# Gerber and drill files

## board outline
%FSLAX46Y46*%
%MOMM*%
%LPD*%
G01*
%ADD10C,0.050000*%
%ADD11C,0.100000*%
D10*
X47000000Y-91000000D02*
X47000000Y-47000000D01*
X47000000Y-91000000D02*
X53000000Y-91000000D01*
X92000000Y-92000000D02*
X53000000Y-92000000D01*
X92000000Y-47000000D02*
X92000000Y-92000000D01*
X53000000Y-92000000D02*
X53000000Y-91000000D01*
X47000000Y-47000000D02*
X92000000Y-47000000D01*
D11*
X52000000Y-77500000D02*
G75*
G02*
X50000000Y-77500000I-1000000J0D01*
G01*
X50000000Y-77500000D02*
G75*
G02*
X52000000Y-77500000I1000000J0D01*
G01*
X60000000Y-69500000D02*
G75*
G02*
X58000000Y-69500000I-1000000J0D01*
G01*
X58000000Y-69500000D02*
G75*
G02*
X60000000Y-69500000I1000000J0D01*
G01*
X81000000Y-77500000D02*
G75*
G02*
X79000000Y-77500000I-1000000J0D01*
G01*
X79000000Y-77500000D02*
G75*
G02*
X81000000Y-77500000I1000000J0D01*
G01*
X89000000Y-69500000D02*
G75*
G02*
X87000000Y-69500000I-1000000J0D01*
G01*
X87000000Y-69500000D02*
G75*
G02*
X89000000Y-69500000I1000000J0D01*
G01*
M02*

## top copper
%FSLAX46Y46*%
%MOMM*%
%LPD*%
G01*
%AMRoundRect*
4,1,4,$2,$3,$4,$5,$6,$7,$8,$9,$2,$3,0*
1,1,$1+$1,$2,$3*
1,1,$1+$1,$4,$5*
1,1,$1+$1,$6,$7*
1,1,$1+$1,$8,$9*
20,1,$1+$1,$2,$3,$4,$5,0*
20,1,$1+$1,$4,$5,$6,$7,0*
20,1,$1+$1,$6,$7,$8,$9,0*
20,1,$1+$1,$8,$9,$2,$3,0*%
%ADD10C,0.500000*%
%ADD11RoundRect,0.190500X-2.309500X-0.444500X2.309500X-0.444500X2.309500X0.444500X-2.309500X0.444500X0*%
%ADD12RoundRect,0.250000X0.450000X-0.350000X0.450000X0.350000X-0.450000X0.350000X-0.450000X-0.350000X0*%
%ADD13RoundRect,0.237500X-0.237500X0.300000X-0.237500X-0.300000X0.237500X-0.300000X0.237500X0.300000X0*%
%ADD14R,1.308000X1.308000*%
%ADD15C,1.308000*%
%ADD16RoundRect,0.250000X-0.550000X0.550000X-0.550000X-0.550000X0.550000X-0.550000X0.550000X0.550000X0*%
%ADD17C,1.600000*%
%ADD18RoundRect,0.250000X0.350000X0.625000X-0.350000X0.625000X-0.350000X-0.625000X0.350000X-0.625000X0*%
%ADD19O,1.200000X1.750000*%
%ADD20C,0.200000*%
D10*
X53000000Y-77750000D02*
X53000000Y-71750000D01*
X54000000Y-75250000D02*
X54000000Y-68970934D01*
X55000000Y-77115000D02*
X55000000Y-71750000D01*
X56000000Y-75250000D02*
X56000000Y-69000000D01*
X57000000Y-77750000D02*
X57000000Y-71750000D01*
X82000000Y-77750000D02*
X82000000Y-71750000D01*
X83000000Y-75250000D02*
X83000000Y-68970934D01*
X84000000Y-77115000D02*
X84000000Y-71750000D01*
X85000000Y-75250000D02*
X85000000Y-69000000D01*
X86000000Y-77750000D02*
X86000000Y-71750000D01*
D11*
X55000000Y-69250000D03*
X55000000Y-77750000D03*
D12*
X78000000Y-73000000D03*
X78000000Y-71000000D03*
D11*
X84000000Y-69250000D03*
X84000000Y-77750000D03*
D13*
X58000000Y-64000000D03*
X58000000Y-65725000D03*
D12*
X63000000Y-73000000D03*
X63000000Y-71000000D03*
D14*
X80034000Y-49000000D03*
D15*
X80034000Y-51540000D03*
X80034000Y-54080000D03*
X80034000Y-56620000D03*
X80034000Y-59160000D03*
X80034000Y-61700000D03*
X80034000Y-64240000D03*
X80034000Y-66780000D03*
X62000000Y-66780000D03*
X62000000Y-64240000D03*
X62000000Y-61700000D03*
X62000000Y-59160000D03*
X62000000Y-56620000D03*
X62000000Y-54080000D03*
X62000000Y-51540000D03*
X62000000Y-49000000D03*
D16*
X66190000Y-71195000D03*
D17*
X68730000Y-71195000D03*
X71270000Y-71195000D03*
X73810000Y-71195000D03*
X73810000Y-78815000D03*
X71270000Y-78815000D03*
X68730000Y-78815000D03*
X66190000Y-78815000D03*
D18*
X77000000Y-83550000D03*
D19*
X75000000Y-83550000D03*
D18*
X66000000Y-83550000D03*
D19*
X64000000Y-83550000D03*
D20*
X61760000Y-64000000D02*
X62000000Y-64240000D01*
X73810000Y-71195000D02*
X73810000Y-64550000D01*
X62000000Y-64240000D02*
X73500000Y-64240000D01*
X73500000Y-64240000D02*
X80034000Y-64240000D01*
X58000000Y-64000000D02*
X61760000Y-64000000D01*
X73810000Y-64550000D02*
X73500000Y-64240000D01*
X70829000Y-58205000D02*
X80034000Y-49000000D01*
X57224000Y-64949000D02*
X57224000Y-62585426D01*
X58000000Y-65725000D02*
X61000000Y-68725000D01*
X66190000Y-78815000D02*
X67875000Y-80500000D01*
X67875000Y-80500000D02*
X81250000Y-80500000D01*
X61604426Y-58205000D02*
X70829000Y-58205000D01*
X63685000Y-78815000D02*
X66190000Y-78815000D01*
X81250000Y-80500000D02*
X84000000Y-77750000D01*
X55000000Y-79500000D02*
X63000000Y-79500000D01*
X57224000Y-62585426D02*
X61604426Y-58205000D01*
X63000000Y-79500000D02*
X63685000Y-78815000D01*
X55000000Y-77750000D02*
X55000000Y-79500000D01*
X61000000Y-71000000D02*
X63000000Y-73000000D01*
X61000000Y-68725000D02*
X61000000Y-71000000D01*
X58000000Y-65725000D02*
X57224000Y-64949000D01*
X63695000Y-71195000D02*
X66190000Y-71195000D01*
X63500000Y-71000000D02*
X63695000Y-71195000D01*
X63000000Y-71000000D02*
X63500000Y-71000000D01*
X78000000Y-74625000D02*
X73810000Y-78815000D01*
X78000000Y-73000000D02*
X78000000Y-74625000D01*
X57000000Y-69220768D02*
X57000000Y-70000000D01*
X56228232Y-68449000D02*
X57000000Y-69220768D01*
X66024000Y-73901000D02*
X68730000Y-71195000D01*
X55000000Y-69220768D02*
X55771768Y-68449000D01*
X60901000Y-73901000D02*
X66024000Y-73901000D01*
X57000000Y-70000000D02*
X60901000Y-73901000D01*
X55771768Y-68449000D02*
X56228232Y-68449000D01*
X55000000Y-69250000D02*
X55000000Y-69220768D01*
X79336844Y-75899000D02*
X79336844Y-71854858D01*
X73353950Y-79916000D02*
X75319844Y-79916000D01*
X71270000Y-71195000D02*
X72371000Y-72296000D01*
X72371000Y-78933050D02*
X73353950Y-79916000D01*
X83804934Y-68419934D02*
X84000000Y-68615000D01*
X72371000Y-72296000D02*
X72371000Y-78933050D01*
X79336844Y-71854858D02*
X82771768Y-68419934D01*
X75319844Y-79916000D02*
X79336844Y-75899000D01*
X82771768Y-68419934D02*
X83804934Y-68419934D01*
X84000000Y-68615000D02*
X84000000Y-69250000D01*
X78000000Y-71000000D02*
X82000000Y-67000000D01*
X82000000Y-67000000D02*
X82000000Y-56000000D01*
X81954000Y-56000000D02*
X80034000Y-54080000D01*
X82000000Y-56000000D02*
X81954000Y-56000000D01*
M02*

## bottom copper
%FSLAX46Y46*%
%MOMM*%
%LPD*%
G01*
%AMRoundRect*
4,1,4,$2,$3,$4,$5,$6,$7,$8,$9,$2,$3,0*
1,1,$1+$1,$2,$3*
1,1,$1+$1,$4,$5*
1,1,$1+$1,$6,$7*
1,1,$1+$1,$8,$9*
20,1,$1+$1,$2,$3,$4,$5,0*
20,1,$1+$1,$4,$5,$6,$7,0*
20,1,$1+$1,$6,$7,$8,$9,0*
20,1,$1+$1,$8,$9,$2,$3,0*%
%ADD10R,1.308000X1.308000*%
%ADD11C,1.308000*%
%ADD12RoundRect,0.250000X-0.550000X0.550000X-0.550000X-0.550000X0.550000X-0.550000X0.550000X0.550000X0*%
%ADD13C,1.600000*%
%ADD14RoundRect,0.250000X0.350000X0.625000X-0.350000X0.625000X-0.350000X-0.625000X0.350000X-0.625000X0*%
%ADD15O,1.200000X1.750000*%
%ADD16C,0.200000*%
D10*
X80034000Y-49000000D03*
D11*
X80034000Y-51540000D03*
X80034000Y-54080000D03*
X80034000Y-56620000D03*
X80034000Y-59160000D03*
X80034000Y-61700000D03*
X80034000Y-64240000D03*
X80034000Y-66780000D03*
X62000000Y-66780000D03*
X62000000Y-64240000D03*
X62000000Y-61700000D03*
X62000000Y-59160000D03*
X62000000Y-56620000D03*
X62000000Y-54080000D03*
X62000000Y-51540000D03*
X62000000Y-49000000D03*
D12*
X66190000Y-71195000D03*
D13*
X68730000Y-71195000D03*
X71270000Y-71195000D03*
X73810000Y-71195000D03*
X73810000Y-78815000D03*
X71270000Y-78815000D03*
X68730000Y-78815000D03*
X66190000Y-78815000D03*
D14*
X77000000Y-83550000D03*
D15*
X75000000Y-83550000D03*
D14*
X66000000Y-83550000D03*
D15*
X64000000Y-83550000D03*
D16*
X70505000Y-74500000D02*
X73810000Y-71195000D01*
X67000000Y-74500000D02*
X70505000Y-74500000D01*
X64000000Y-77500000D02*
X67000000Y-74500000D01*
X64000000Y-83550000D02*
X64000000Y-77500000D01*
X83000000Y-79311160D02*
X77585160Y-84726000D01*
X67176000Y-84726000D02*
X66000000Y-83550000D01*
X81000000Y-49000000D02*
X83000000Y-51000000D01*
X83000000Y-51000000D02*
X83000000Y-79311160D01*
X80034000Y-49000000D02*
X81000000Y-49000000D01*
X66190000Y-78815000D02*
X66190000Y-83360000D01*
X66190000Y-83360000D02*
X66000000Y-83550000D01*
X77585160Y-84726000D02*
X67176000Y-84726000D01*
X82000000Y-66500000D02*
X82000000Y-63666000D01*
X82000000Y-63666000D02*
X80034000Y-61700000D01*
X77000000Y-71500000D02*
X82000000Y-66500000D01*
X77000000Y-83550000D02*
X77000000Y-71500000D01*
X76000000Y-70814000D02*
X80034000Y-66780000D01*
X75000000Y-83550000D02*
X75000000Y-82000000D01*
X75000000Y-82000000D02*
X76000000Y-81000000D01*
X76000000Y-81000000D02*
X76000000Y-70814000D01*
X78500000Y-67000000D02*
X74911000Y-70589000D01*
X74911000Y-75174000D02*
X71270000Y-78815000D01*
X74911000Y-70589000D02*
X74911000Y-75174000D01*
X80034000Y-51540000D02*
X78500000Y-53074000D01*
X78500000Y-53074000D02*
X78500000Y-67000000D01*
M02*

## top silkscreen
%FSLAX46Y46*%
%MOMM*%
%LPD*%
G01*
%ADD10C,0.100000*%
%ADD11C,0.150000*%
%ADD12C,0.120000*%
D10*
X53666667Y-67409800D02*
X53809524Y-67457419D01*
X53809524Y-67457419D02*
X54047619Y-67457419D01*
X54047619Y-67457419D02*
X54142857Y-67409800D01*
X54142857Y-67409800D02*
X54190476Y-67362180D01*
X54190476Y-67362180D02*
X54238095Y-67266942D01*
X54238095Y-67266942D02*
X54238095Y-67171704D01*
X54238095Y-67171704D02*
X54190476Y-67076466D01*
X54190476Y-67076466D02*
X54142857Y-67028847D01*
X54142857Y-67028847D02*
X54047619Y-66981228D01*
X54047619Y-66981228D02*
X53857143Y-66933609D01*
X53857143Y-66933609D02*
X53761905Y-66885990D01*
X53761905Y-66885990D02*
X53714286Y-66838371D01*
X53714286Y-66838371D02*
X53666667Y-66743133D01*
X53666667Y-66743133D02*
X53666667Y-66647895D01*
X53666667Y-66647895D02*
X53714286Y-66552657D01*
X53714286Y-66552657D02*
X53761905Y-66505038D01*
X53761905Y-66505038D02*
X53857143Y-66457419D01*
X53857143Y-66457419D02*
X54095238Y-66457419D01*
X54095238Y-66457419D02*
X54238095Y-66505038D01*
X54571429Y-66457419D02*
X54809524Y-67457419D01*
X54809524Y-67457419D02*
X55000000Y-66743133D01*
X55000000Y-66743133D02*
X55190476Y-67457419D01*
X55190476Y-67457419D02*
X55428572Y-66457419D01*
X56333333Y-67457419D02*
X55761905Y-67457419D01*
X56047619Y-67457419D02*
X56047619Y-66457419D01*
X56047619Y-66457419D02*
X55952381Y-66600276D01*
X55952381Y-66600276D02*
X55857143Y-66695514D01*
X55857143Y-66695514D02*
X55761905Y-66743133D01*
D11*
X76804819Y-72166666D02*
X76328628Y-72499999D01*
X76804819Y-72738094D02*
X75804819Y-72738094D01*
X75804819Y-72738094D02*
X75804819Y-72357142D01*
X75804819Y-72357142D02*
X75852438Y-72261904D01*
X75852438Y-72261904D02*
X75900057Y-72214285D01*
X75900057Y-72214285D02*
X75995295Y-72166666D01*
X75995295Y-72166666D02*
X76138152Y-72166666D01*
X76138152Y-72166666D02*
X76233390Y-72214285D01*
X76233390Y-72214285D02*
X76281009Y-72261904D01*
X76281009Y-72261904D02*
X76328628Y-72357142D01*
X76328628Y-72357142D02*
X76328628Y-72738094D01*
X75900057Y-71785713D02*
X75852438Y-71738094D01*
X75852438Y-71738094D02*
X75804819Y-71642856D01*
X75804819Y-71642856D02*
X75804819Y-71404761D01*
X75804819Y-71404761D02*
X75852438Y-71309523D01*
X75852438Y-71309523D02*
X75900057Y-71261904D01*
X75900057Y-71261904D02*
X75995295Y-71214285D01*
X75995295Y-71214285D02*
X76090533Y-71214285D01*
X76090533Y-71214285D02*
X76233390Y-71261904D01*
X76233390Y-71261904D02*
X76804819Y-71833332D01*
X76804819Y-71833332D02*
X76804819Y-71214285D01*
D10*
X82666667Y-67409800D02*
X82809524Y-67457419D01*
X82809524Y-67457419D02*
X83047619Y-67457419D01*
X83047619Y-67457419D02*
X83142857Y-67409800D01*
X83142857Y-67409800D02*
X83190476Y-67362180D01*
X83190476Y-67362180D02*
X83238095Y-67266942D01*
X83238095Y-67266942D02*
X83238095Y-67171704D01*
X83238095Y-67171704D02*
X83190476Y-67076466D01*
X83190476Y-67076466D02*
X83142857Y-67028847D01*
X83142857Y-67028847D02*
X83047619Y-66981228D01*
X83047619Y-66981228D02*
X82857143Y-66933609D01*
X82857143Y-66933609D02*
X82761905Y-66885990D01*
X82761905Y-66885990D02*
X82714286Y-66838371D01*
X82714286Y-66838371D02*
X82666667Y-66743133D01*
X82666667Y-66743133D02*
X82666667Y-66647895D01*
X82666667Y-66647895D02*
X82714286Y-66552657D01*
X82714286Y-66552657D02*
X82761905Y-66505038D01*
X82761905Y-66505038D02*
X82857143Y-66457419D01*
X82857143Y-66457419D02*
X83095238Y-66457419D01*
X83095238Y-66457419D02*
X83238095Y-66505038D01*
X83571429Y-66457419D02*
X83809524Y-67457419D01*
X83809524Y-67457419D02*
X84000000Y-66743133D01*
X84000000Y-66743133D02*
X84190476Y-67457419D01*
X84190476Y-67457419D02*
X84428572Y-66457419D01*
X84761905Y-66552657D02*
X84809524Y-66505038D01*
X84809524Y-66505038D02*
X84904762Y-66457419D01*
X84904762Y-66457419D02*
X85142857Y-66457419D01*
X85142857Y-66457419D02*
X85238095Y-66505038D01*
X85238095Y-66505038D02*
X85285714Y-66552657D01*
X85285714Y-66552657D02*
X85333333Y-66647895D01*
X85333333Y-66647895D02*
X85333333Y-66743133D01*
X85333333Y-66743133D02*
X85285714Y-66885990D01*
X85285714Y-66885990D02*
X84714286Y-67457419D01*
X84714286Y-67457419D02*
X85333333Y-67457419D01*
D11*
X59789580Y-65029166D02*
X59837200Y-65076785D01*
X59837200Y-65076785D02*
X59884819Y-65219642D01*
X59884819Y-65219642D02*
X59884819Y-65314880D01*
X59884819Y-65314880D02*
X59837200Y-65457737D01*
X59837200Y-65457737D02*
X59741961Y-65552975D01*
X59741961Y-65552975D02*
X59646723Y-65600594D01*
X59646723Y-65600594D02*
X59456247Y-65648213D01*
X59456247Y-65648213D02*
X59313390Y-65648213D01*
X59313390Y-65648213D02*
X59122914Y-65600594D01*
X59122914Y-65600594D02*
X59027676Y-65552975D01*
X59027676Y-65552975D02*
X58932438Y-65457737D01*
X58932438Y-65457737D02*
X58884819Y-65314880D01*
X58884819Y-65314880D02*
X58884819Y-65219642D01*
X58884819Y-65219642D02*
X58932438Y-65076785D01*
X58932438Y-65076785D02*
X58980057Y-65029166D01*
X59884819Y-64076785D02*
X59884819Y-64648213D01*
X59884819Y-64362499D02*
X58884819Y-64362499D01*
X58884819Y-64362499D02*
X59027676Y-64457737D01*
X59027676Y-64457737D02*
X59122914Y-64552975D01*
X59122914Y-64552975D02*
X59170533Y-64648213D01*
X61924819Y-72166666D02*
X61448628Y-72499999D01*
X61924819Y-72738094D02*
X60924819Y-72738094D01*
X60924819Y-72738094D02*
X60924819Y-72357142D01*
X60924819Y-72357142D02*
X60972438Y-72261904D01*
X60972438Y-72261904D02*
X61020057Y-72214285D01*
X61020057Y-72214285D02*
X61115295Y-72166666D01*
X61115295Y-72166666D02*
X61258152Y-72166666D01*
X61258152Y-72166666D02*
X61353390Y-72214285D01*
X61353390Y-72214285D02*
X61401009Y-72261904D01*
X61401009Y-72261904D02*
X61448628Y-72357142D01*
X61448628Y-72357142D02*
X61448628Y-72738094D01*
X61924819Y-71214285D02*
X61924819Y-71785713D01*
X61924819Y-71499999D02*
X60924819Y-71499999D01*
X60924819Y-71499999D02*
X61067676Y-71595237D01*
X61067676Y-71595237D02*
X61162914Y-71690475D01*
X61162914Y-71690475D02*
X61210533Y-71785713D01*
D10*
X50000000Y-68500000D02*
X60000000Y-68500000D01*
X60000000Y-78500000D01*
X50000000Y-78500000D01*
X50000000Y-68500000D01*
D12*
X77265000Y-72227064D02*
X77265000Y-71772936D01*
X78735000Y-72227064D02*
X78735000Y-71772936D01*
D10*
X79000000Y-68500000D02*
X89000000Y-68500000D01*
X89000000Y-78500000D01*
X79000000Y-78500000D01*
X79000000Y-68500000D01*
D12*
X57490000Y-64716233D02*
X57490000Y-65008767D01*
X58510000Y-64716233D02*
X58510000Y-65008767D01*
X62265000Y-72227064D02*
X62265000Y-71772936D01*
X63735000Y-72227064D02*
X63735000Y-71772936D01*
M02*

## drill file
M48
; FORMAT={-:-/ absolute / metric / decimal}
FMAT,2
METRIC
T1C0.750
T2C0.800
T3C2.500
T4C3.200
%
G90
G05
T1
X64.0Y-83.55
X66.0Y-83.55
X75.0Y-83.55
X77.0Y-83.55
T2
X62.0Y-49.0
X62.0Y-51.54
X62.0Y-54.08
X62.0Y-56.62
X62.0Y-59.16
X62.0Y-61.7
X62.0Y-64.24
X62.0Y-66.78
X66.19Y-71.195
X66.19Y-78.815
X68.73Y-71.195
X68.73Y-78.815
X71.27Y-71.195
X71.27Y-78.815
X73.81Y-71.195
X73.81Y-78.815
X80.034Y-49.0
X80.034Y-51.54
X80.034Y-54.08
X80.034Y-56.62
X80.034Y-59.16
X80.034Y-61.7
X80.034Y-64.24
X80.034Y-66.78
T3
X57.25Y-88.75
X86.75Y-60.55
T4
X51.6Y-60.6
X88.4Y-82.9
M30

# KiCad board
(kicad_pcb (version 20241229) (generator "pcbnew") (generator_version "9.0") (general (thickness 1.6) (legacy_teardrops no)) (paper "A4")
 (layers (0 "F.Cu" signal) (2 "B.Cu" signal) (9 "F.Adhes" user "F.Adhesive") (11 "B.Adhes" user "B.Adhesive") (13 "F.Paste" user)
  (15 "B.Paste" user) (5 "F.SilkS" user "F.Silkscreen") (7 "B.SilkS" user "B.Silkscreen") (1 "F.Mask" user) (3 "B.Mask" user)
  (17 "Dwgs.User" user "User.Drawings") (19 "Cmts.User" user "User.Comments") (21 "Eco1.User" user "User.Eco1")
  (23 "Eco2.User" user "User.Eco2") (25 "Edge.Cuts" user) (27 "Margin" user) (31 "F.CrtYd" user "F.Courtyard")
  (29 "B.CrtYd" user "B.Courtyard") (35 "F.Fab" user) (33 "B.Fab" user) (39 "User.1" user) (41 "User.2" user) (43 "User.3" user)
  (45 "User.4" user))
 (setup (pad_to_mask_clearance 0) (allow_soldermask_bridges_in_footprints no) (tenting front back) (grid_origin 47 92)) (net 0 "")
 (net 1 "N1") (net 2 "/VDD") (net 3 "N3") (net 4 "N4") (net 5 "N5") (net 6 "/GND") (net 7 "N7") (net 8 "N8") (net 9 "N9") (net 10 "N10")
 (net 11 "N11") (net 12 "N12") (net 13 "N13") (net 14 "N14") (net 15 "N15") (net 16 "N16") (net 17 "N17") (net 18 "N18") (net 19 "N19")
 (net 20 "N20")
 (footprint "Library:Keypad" (layer "F.Cu") (at 50 78.5)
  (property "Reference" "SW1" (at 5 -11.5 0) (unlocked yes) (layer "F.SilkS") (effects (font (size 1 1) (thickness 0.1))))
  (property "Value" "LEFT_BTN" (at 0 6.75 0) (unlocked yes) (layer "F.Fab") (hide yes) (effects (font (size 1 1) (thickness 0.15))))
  (fp_line (start 3 -0.75) (end 3 -6.75) (stroke (width 0.5) (type solid)) (layer "F.Cu"))
  (fp_line (start 4 -3.25) (end 4 -9.529066) (stroke (width 0.5) (type solid)) (layer "F.Cu"))
  (fp_line (start 5 -1.385) (end 5 -6.75) (stroke (width 0.5) (type solid)) (layer "F.Cu"))
  (fp_line (start 6 -3.25) (end 6 -9.5) (stroke (width 0.5) (type solid)) (layer "F.Cu"))
  (fp_line (start 7 -0.75) (end 7 -6.75) (stroke (width 0.5) (type solid)) (layer "F.Cu"))
  (fp_rect (start 0 -10) (end 10 0) (stroke (width 0.1) (type default)) (fill no) (layer "F.SilkS"))
  (fp_circle (center 1 -1) (end 0 -1) (stroke (width 0.1) (type solid)) (fill no) (layer "Edge.Cuts"))
  (fp_circle (center 9 -9) (end 10 -9) (stroke (width 0.1) (type solid)) (fill no) (layer "Edge.Cuts"))
  (pad "1" smd roundrect (at 5 -9.25) (size 5 1.27) (layers "F.Cu") (roundrect_rratio 0.15) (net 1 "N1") (thermal_bridge_angle 45))
  (pad "2" smd roundrect (at 5 -0.75) (size 5 1.27) (layers "F.Cu") (roundrect_rratio 0.15) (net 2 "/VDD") (thermal_bridge_angle 45)))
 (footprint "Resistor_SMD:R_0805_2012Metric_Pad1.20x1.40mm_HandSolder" (layer "F.Cu") (at 78 72 90)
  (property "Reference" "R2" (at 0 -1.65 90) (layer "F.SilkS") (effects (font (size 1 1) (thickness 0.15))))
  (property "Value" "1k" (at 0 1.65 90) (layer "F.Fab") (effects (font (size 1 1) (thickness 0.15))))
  (fp_line (start -0.227064 -0.735) (end 0.227064 -0.735) (stroke (width 0.12) (type solid)) (layer "F.SilkS"))
  (fp_line (start -0.227064 0.735) (end 0.227064 0.735) (stroke (width 0.12) (type solid)) (layer "F.SilkS"))
  (pad "1" smd roundrect (at -1 0 90) (size 1.2 1.4) (layers "F.Cu" "F.Mask" "F.Paste") (roundrect_rratio 0.208333) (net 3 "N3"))
  (pad "2" smd roundrect (at 1 0 90) (size 1.2 1.4) (layers "F.Cu" "F.Mask" "F.Paste") (roundrect_rratio 0.208333) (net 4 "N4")))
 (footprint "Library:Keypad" (layer "F.Cu") (at 79 78.5)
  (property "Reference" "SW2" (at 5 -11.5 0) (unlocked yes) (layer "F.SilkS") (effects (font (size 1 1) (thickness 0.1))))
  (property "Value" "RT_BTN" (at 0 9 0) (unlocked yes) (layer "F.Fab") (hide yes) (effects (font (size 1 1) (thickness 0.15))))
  (fp_line (start 3 -0.75) (end 3 -6.75) (stroke (width 0.5) (type solid)) (layer "F.Cu"))
  (fp_line (start 4 -3.25) (end 4 -9.529066) (stroke (width 0.5) (type solid)) (layer "F.Cu"))
  (fp_line (start 5 -1.385) (end 5 -6.75) (stroke (width 0.5) (type solid)) (layer "F.Cu"))
  (fp_line (start 6 -3.25) (end 6 -9.5) (stroke (width 0.5) (type solid)) (layer "F.Cu"))
  (fp_line (start 7 -0.75) (end 7 -6.75) (stroke (width 0.5) (type solid)) (layer "F.Cu"))
  (fp_rect (start 0 -10) (end 10 0) (stroke (width 0.1) (type default)) (fill no) (layer "F.SilkS"))
  (fp_circle (center 1 -1) (end 0 -1) (stroke (width 0.1) (type solid)) (fill no) (layer "Edge.Cuts"))
  (fp_circle (center 9 -9) (end 10 -9) (stroke (width 0.1) (type solid)) (fill no) (layer "Edge.Cuts"))
  (pad "1" smd roundrect (at 5 -9.25) (size 5 1.27) (layers "F.Cu") (roundrect_rratio 0.15) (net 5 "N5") (thermal_bridge_angle 45))
  (pad "2" smd roundrect (at 5 -0.75) (size 5 1.27) (layers "F.Cu") (roundrect_rratio 0.15) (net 2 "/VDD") (thermal_bridge_angle 45)))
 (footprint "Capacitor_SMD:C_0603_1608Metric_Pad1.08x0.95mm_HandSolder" (layer "F.Cu") (at 58 64.8625 -90)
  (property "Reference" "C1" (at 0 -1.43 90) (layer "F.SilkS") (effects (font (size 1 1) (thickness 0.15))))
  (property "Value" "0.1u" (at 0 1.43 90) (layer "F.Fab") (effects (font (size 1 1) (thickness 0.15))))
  (fp_line (start -0.146267 0.51) (end 0.146267 0.51) (stroke (width 0.12) (type solid)) (layer "F.SilkS"))
  (fp_line (start -0.146267 -0.51) (end 0.146267 -0.51) (stroke (width 0.12) (type solid)) (layer "F.SilkS"))
  (pad "1" smd roundrect (at -0.8625 0 270) (size 1.075 0.95) (layers "F.Cu" "F.Mask" "F.Paste") (roundrect_rratio 0.25) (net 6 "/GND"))
  (pad "2" smd roundrect (at 0.8625 0 270) (size 1.075 0.95) (layers "F.Cu" "F.Mask" "F.Paste") (roundrect_rratio 0.25) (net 2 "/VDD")))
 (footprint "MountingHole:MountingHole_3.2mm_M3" (layer "F.Cu") (at 51.6 60.6)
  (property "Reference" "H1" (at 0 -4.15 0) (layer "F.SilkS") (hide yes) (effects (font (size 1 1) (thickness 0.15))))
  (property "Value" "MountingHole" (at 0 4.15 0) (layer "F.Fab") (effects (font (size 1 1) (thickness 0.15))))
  (pad "" np_thru_hole circle (at 0 0) (size 3.2 3.2) (drill 3.2) (layers "*.Cu" "*.Mask")))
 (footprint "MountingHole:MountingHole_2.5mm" (layer "F.Cu") (at 86.75 60.55)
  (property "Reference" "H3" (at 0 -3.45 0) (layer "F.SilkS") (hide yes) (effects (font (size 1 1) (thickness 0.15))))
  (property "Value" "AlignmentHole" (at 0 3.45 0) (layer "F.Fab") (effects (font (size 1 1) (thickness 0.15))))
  (pad "" np_thru_hole circle (at 0 0) (size 2.5 2.5) (drill 2.5) (layers "*.Cu" "*.Mask")))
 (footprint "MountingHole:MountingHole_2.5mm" (layer "F.Cu") (at 57.25 88.75)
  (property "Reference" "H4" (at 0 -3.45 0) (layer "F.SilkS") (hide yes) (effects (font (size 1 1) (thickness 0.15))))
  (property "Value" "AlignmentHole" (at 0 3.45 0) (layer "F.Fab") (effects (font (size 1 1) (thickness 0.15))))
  (pad "" np_thru_hole circle (at 0 0) (size 2.5 2.5) (drill 2.5) (layers "*.Cu" "*.Mask")))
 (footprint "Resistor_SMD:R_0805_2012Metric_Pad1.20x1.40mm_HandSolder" (layer "F.Cu") (at 63 72 90)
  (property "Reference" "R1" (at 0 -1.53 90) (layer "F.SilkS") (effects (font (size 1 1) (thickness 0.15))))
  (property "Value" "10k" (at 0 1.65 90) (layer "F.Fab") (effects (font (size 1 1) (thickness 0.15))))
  (fp_line (start -0.227064 -0.735) (end 0.227064 -0.735) (stroke (width 0.12) (type solid)) (layer "F.SilkS"))
  (fp_line (start -0.227064 0.735) (end 0.227064 0.735) (stroke (width 0.12) (type solid)) (layer "F.SilkS"))
  (pad "1" smd roundrect (at -1 0 90) (size 1.2 1.4) (layers "F.Cu" "F.Mask" "F.Paste") (roundrect_rratio 0.208333) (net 2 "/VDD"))
  (pad "2" smd roundrect (at 1 0 90) (size 1.2 1.4) (layers "F.Cu" "F.Mask" "F.Paste") (roundrect_rratio 0.208333) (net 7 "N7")))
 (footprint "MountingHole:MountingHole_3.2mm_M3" (layer "F.Cu") (at 88.4 82.9)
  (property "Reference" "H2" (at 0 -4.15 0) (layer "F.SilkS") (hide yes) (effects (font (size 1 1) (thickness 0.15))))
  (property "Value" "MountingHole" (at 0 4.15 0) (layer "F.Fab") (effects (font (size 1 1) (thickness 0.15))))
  (pad "" np_thru_hole circle (at 0 0) (size 3.2 3.2) (drill 3.2) (layers "*.Cu" "*.Mask")))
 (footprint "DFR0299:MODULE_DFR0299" (layer "B.Cu") (at 71.017 57.89 180)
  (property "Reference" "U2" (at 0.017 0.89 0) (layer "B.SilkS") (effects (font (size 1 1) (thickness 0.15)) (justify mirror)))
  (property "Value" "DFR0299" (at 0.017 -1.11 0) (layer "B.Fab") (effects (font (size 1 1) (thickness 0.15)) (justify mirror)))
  (pad "1" thru_hole rect (at -9.017 8.89 180) (size 1.308 1.308) (drill 0.8) (layers "*.Cu" "*.Mask") (remove_unused_layers no)
   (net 2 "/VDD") (solder_mask_margin 0.102))
  (pad "2" thru_hole circle (at -9.017 6.35 180) (size 1.308 1.308) (drill 0.8) (layers "*.Cu" "*.Mask") (remove_unused_layers no)
   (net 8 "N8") (solder_mask_margin 0.102))
  (pad "3" thru_hole circle (at -9.017 3.81 180) (size 1.308 1.308) (drill 0.8) (layers "*.Cu" "*.Mask") (remove_unused_layers no)
   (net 4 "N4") (solder_mask_margin 0.102))
  (pad "4" thru_hole circle (at -9.017 1.27 180) (size 1.308 1.308) (drill 0.8) (layers "*.Cu" "*.Mask") (remove_unused_layers no)
   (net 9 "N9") (solder_mask_margin 0.102))
  (pad "5" thru_hole circle (at -9.017 -1.27 180) (size 1.308 1.308) (drill 0.8) (layers "*.Cu" "*.Mask") (remove_unused_layers no)
   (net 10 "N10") (solder_mask_margin 0.102))
  (pad "6" thru_hole circle (at -9.017 -3.81 180) (size 1.308 1.308) (drill 0.8) (layers "*.Cu" "*.Mask") (remove_unused_layers no)
   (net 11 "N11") (solder_mask_margin 0.102))
  (pad "7" thru_hole circle (at -9.017 -6.35 180) (size 1.308 1.308) (drill 0.8) (layers "*.Cu" "*.Mask") (remove_unused_layers no)
   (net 6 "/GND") (solder_mask_margin 0.102))
  (pad "8" thru_hole circle (at -9.017 -8.89 180) (size 1.308 1.308) (drill 0.8) (layers "*.Cu" "*.Mask") (remove_unused_layers no)
   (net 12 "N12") (solder_mask_margin 0.102))
  (pad "9" thru_hole circle (at 9.017 -8.89 180) (size 1.308 1.308) (drill 0.8) (layers "*.Cu" "*.Mask") (remove_unused_layers no)
   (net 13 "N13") (solder_mask_margin 0.102))
  (pad "10" thru_hole circle (at 9.017 -6.35 180) (size 1.308 1.308) (drill 0.8) (layers "*.Cu" "*.Mask") (remove_unused_layers no)
   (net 6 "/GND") (solder_mask_margin 0.102))
  (pad "11" thru_hole circle (at 9.017 -3.81 180) (size 1.308 1.308) (drill 0.8) (layers "*.Cu" "*.Mask") (remove_unused_layers no)
   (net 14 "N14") (solder_mask_margin 0.102))
  (pad "12" thru_hole circle (at 9.017 -1.27 180) (size 1.308 1.308) (drill 0.8) (layers "*.Cu" "*.Mask") (remove_unused_layers no)
   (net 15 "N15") (solder_mask_margin 0.102))
  (pad "13" thru_hole circle (at 9.017 1.27 180) (size 1.308 1.308) (drill 0.8) (layers "*.Cu" "*.Mask") (remove_unused_layers no)
   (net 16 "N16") (solder_mask_margin 0.102))
  (pad "14" thru_hole circle (at 9.017 3.81 180) (size 1.308 1.308) (drill 0.8) (layers "*.Cu" "*.Mask") (remove_unused_layers no)
   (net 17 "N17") (solder_mask_margin 0.102))
  (pad "15" thru_hole circle (at 9.017 6.35 180) (size 1.308 1.308) (drill 0.8) (layers "*.Cu" "*.Mask") (remove_unused_layers no)
   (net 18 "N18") (solder_mask_margin 0.102))
  (pad "16" thru_hole circle (at 9.017 8.89 180) (size 1.308 1.308) (drill 0.8) (layers "*.Cu" "*.Mask") (remove_unused_layers no)
   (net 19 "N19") (solder_mask_margin 0.102)))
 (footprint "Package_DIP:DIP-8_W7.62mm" (layer "B.Cu") (at 66.19 71.195 -90)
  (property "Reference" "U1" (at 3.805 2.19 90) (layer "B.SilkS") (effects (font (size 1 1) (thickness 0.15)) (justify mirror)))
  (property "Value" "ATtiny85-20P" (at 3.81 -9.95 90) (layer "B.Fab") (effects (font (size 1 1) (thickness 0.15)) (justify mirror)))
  (pad "1" thru_hole roundrect (at 0 0 270) (size 1.6 1.6) (drill 0.8) (layers "*.Cu" "*.Mask") (remove_unused_layers no)
   (roundrect_rratio 0.15625) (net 7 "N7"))
  (pad "2" thru_hole circle (at 0 -2.54 270) (size 1.6 1.6) (drill 0.8) (layers "*.Cu" "*.Mask") (remove_unused_layers no) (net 1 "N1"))
  (pad "3" thru_hole circle (at 0 -5.08 270) (size 1.6 1.6) (drill 0.8) (layers "*.Cu" "*.Mask") (remove_unused_layers no) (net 5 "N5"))
  (pad "4" thru_hole circle (at 0 -7.62 270) (size 1.6 1.6) (drill 0.8) (layers "*.Cu" "*.Mask") (remove_unused_layers no) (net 6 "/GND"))
  (pad "5" thru_hole circle (at 7.62 -7.62 270) (size 1.6 1.6) (drill 0.8) (layers "*.Cu" "*.Mask") (remove_unused_layers no) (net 3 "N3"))
  (pad "6" thru_hole circle (at 7.62 -5.08 270) (size 1.6 1.6) (drill 0.8) (layers "*.Cu" "*.Mask") (remove_unused_layers no) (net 8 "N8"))
  (pad "7" thru_hole circle (at 7.62 -2.54 270) (size 1.6 1.6) (drill 0.8) (layers "*.Cu" "*.Mask") (remove_unused_layers no) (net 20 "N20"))
  (pad "8" thru_hole circle (at 7.62 0 270) (size 1.6 1.6) (drill 0.8) (layers "*.Cu" "*.Mask") (remove_unused_layers no) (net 2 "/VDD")))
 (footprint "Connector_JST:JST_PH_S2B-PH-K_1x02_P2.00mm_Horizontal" (layer "B.Cu") (at 77 83.55 180)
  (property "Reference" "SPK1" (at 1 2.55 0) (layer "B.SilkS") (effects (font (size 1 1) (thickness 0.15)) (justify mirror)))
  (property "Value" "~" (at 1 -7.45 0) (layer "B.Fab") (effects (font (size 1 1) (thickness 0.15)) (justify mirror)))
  (pad "1" thru_hole roundrect (at 0 0 180) (size 1.2 1.75) (drill 0.75) (layers "*.Cu" "*.Mask") (remove_unused_layers no)
   (roundrect_rratio 0.208333) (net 11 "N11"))
  (pad "2" thru_hole oval (at 2 0 180) (size 1.2 1.75) (drill 0.75) (layers "*.Cu" "*.Mask") (remove_unused_layers no) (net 12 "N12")))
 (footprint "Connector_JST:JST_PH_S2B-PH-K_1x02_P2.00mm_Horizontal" (layer "B.Cu") (at 66 83.55 180)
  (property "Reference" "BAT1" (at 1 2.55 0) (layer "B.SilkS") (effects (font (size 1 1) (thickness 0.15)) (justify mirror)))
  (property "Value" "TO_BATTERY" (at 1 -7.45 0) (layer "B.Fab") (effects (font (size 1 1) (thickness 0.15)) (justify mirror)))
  (pad "1" thru_hole roundrect (at 0 0 180) (size 1.2 1.75) (drill 0.75) (layers "*.Cu" "*.Mask") (remove_unused_layers no)
   (roundrect_rratio 0.208333) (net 2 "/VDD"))
  (pad "2" thru_hole oval (at 2 0 180) (size 1.2 1.75) (drill 0.75) (layers "*.Cu" "*.Mask") (remove_unused_layers no) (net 6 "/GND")))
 (gr_line (start 47 91) (end 47 47) (stroke (width 0.05) (type default)) (layer "Edge.Cuts"))
 (gr_line (start 47 91) (end 53 91) (stroke (width 0.05) (type default)) (layer "Edge.Cuts"))
 (gr_line (start 92 92) (end 53 92) (stroke (width 0.05) (type default)) (layer "Edge.Cuts"))
 (gr_line (start 92 47) (end 92 92) (stroke (width 0.05) (type default)) (layer "Edge.Cuts"))
 (gr_line (start 53 92) (end 53 91) (stroke (width 0.05) (type default)) (layer "Edge.Cuts"))
 (gr_line (start 47 47) (end 92 47) (stroke (width 0.05) (type default)) (layer "Edge.Cuts"))
 (segment (start 61.76 64) (end 62 64.24) (width 0.2) (layer "F.Cu") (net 6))
 (segment (start 73.81 71.195) (end 73.81 64.55) (width 0.2) (layer "F.Cu") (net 6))
 (segment (start 62 64.24) (end 73.5 64.24) (width 0.2) (layer "F.Cu") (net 6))
 (segment (start 73.5 64.24) (end 80.034 64.24) (width 0.2) (layer "F.Cu") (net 6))
 (segment (start 58 64) (end 61.76 64) (width 0.2) (layer "F.Cu") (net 6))
 (segment (start 73.81 64.55) (end 73.5 64.24) (width 0.2) (layer "F.Cu") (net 6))
 (segment (start 70.505 74.5) (end 73.81 71.195) (width 0.2) (layer "B.Cu") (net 6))
 (segment (start 67 74.5) (end 70.505 74.5) (width 0.2) (layer "B.Cu") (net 6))
 (segment (start 64 77.5) (end 67 74.5) (width 0.2) (layer "B.Cu") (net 6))
 (segment (start 64 83.55) (end 64 77.5) (width 0.2) (layer "B.Cu") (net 6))
 (segment (start 70.829 58.205) (end 80.034 49) (width 0.2) (layer "F.Cu") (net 2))
 (segment (start 57.224 64.949) (end 57.224 62.585426) (width 0.2) (layer "F.Cu") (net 2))
 (segment (start 58 65.725) (end 61 68.725) (width 0.2) (layer "F.Cu") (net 2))
 (segment (start 66.19 78.815) (end 67.875 80.5) (width 0.2) (layer "F.Cu") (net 2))
 (segment (start 67.875 80.5) (end 81.25 80.5) (width 0.2) (layer "F.Cu") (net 2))
 (segment (start 61.604426 58.205) (end 70.829 58.205) (width 0.2) (layer "F.Cu") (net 2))
 (segment (start 63.685 78.815) (end 66.19 78.815) (width 0.2) (layer "F.Cu") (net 2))
 (segment (start 81.25 80.5) (end 84 77.75) (width 0.2) (layer "F.Cu") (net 2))
 (segment (start 55 79.5) (end 63 79.5) (width 0.2) (layer "F.Cu") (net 2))
 (segment (start 57.224 62.585426) (end 61.604426 58.205) (width 0.2) (layer "F.Cu") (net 2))
 (segment (start 63 79.5) (end 63.685 78.815) (width 0.2) (layer "F.Cu") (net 2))
 (segment (start 55 77.75) (end 55 79.5) (width 0.2) (layer "F.Cu") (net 2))
 (segment (start 61 71) (end 63 73) (width 0.2) (layer "F.Cu") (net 2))
 (segment (start 61 68.725) (end 61 71) (width 0.2) (layer "F.Cu") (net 2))
 (segment (start 58 65.725) (end 57.224 64.949) (width 0.2) (layer "F.Cu") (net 2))
 (segment (start 83 79.31116) (end 77.58516 84.726) (width 0.2) (layer "B.Cu") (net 2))
 (segment (start 67.176 84.726) (end 66 83.55) (width 0.2) (layer "B.Cu") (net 2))
 (segment (start 81 49) (end 83 51) (width 0.2) (layer "B.Cu") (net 2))
 (segment (start 83 51) (end 83 79.31116) (width 0.2) (layer "B.Cu") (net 2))
 (segment (start 80.034 49) (end 81 49) (width 0.2) (layer "B.Cu") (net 2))
 (segment (start 66.19 78.815) (end 66.19 83.36) (width 0.2) (layer "B.Cu") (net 2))
 (segment (start 66.19 83.36) (end 66 83.55) (width 0.2) (layer "B.Cu") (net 2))
 (segment (start 77.58516 84.726) (end 67.176 84.726) (width 0.2) (layer "B.Cu") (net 2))
 (segment (start 63.695 71.195) (end 66.19 71.195) (width 0.2) (layer "F.Cu") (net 7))
 (segment (start 63.5 71) (end 63.695 71.195) (width 0.2) (layer "F.Cu") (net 7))
 (segment (start 63 71) (end 63.5 71) (width 0.2) (layer "F.Cu") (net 7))
 (segment (start 78 74.625) (end 73.81 78.815) (width 0.2) (layer "F.Cu") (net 3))
 (segment (start 78 73) (end 78 74.625) (width 0.2) (layer "F.Cu") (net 3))
 (segment (start 82 66.5) (end 82 63.666) (width 0.2) (layer "B.Cu") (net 11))
 (segment (start 82 63.666) (end 80.034 61.7) (width 0.2) (layer "B.Cu") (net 11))
 (segment (start 77 71.5) (end 82 66.5) (width 0.2) (layer "B.Cu") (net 11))
 (segment (start 77 83.55) (end 77 71.5) (width 0.2) (layer "B.Cu") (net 11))
 (segment (start 76 70.814) (end 80.034 66.78) (width 0.2) (layer "B.Cu") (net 12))
 (segment (start 75 83.55) (end 75 82) (width 0.2) (layer "B.Cu") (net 12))
 (segment (start 75 82) (end 76 81) (width 0.2) (layer "B.Cu") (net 12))
 (segment (start 76 81) (end 76 70.814) (width 0.2) (layer "B.Cu") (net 12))
 (segment (start 78.5 67) (end 74.911 70.589) (width 0.2) (layer "B.Cu") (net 8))
 (segment (start 74.911 75.174) (end 71.27 78.815) (width 0.2) (layer "B.Cu") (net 8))
 (segment (start 74.911 70.589) (end 74.911 75.174) (width 0.2) (layer "B.Cu") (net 8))
 (segment (start 80.034 51.54) (end 78.5 53.074) (width 0.2) (layer "B.Cu") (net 8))
 (segment (start 78.5 53.074) (end 78.5 67) (width 0.2) (layer "B.Cu") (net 8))
 (segment (start 57 69.220768) (end 57 70) (width 0.2) (layer "F.Cu") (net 1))
 (segment (start 56.228232 68.449) (end 57 69.220768) (width 0.2) (layer "F.Cu") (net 1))
 (segment (start 66.024 73.901) (end 68.73 71.195) (width 0.2) (layer "F.Cu") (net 1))
 (segment (start 55 69.220768) (end 55.771768 68.449) (width 0.2) (layer "F.Cu") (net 1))
 (segment (start 60.901 73.901) (end 66.024 73.901) (width 0.2) (layer "F.Cu") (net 1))
 (segment (start 57 70) (end 60.901 73.901) (width 0.2) (layer "F.Cu") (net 1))
 (segment (start 55.771768 68.449) (end 56.228232 68.449) (width 0.2) (layer "F.Cu") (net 1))
 (segment (start 55 69.25) (end 55 69.220768) (width 0.2) (layer "F.Cu") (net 1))
 (segment (start 79.336844 75.899) (end 79.336844 71.854858) (width 0.2) (layer "F.Cu") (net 5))
 (segment (start 73.35395 79.916) (end 75.319844 79.916) (width 0.2) (layer "F.Cu") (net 5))
 (segment (start 71.27 71.195) (end 72.371 72.296) (width 0.2) (layer "F.Cu") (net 5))
 (segment (start 72.371 78.93305) (end 73.35395 79.916) (width 0.2) (layer "F.Cu") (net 5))
 (segment (start 83.804934 68.419934) (end 84 68.615) (width 0.2) (layer "F.Cu") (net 5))
 (segment (start 72.371 72.296) (end 72.371 78.93305) (width 0.2) (layer "F.Cu") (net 5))
 (segment (start 79.336844 71.854858) (end 82.771768 68.419934) (width 0.2) (layer "F.Cu") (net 5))
 (segment (start 75.319844 79.916) (end 79.336844 75.899) (width 0.2) (layer "F.Cu") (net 5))
 (segment (start 82.771768 68.419934) (end 83.804934 68.419934) (width 0.2) (layer "F.Cu") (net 5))
 (segment (start 84 68.615) (end 84 69.25) (width 0.2) (layer "F.Cu") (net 5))
 (segment (start 78 71) (end 82 67) (width 0.2) (layer "F.Cu") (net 4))
 (segment (start 82 67) (end 82 56) (width 0.2) (layer "F.Cu") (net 4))
 (segment (start 81.954 56) (end 80.034 54.08) (width 0.2) (layer "F.Cu") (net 4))
 (segment (start 82 56) (end 81.954 56) (width 0.2) (layer "F.Cu") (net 4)))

